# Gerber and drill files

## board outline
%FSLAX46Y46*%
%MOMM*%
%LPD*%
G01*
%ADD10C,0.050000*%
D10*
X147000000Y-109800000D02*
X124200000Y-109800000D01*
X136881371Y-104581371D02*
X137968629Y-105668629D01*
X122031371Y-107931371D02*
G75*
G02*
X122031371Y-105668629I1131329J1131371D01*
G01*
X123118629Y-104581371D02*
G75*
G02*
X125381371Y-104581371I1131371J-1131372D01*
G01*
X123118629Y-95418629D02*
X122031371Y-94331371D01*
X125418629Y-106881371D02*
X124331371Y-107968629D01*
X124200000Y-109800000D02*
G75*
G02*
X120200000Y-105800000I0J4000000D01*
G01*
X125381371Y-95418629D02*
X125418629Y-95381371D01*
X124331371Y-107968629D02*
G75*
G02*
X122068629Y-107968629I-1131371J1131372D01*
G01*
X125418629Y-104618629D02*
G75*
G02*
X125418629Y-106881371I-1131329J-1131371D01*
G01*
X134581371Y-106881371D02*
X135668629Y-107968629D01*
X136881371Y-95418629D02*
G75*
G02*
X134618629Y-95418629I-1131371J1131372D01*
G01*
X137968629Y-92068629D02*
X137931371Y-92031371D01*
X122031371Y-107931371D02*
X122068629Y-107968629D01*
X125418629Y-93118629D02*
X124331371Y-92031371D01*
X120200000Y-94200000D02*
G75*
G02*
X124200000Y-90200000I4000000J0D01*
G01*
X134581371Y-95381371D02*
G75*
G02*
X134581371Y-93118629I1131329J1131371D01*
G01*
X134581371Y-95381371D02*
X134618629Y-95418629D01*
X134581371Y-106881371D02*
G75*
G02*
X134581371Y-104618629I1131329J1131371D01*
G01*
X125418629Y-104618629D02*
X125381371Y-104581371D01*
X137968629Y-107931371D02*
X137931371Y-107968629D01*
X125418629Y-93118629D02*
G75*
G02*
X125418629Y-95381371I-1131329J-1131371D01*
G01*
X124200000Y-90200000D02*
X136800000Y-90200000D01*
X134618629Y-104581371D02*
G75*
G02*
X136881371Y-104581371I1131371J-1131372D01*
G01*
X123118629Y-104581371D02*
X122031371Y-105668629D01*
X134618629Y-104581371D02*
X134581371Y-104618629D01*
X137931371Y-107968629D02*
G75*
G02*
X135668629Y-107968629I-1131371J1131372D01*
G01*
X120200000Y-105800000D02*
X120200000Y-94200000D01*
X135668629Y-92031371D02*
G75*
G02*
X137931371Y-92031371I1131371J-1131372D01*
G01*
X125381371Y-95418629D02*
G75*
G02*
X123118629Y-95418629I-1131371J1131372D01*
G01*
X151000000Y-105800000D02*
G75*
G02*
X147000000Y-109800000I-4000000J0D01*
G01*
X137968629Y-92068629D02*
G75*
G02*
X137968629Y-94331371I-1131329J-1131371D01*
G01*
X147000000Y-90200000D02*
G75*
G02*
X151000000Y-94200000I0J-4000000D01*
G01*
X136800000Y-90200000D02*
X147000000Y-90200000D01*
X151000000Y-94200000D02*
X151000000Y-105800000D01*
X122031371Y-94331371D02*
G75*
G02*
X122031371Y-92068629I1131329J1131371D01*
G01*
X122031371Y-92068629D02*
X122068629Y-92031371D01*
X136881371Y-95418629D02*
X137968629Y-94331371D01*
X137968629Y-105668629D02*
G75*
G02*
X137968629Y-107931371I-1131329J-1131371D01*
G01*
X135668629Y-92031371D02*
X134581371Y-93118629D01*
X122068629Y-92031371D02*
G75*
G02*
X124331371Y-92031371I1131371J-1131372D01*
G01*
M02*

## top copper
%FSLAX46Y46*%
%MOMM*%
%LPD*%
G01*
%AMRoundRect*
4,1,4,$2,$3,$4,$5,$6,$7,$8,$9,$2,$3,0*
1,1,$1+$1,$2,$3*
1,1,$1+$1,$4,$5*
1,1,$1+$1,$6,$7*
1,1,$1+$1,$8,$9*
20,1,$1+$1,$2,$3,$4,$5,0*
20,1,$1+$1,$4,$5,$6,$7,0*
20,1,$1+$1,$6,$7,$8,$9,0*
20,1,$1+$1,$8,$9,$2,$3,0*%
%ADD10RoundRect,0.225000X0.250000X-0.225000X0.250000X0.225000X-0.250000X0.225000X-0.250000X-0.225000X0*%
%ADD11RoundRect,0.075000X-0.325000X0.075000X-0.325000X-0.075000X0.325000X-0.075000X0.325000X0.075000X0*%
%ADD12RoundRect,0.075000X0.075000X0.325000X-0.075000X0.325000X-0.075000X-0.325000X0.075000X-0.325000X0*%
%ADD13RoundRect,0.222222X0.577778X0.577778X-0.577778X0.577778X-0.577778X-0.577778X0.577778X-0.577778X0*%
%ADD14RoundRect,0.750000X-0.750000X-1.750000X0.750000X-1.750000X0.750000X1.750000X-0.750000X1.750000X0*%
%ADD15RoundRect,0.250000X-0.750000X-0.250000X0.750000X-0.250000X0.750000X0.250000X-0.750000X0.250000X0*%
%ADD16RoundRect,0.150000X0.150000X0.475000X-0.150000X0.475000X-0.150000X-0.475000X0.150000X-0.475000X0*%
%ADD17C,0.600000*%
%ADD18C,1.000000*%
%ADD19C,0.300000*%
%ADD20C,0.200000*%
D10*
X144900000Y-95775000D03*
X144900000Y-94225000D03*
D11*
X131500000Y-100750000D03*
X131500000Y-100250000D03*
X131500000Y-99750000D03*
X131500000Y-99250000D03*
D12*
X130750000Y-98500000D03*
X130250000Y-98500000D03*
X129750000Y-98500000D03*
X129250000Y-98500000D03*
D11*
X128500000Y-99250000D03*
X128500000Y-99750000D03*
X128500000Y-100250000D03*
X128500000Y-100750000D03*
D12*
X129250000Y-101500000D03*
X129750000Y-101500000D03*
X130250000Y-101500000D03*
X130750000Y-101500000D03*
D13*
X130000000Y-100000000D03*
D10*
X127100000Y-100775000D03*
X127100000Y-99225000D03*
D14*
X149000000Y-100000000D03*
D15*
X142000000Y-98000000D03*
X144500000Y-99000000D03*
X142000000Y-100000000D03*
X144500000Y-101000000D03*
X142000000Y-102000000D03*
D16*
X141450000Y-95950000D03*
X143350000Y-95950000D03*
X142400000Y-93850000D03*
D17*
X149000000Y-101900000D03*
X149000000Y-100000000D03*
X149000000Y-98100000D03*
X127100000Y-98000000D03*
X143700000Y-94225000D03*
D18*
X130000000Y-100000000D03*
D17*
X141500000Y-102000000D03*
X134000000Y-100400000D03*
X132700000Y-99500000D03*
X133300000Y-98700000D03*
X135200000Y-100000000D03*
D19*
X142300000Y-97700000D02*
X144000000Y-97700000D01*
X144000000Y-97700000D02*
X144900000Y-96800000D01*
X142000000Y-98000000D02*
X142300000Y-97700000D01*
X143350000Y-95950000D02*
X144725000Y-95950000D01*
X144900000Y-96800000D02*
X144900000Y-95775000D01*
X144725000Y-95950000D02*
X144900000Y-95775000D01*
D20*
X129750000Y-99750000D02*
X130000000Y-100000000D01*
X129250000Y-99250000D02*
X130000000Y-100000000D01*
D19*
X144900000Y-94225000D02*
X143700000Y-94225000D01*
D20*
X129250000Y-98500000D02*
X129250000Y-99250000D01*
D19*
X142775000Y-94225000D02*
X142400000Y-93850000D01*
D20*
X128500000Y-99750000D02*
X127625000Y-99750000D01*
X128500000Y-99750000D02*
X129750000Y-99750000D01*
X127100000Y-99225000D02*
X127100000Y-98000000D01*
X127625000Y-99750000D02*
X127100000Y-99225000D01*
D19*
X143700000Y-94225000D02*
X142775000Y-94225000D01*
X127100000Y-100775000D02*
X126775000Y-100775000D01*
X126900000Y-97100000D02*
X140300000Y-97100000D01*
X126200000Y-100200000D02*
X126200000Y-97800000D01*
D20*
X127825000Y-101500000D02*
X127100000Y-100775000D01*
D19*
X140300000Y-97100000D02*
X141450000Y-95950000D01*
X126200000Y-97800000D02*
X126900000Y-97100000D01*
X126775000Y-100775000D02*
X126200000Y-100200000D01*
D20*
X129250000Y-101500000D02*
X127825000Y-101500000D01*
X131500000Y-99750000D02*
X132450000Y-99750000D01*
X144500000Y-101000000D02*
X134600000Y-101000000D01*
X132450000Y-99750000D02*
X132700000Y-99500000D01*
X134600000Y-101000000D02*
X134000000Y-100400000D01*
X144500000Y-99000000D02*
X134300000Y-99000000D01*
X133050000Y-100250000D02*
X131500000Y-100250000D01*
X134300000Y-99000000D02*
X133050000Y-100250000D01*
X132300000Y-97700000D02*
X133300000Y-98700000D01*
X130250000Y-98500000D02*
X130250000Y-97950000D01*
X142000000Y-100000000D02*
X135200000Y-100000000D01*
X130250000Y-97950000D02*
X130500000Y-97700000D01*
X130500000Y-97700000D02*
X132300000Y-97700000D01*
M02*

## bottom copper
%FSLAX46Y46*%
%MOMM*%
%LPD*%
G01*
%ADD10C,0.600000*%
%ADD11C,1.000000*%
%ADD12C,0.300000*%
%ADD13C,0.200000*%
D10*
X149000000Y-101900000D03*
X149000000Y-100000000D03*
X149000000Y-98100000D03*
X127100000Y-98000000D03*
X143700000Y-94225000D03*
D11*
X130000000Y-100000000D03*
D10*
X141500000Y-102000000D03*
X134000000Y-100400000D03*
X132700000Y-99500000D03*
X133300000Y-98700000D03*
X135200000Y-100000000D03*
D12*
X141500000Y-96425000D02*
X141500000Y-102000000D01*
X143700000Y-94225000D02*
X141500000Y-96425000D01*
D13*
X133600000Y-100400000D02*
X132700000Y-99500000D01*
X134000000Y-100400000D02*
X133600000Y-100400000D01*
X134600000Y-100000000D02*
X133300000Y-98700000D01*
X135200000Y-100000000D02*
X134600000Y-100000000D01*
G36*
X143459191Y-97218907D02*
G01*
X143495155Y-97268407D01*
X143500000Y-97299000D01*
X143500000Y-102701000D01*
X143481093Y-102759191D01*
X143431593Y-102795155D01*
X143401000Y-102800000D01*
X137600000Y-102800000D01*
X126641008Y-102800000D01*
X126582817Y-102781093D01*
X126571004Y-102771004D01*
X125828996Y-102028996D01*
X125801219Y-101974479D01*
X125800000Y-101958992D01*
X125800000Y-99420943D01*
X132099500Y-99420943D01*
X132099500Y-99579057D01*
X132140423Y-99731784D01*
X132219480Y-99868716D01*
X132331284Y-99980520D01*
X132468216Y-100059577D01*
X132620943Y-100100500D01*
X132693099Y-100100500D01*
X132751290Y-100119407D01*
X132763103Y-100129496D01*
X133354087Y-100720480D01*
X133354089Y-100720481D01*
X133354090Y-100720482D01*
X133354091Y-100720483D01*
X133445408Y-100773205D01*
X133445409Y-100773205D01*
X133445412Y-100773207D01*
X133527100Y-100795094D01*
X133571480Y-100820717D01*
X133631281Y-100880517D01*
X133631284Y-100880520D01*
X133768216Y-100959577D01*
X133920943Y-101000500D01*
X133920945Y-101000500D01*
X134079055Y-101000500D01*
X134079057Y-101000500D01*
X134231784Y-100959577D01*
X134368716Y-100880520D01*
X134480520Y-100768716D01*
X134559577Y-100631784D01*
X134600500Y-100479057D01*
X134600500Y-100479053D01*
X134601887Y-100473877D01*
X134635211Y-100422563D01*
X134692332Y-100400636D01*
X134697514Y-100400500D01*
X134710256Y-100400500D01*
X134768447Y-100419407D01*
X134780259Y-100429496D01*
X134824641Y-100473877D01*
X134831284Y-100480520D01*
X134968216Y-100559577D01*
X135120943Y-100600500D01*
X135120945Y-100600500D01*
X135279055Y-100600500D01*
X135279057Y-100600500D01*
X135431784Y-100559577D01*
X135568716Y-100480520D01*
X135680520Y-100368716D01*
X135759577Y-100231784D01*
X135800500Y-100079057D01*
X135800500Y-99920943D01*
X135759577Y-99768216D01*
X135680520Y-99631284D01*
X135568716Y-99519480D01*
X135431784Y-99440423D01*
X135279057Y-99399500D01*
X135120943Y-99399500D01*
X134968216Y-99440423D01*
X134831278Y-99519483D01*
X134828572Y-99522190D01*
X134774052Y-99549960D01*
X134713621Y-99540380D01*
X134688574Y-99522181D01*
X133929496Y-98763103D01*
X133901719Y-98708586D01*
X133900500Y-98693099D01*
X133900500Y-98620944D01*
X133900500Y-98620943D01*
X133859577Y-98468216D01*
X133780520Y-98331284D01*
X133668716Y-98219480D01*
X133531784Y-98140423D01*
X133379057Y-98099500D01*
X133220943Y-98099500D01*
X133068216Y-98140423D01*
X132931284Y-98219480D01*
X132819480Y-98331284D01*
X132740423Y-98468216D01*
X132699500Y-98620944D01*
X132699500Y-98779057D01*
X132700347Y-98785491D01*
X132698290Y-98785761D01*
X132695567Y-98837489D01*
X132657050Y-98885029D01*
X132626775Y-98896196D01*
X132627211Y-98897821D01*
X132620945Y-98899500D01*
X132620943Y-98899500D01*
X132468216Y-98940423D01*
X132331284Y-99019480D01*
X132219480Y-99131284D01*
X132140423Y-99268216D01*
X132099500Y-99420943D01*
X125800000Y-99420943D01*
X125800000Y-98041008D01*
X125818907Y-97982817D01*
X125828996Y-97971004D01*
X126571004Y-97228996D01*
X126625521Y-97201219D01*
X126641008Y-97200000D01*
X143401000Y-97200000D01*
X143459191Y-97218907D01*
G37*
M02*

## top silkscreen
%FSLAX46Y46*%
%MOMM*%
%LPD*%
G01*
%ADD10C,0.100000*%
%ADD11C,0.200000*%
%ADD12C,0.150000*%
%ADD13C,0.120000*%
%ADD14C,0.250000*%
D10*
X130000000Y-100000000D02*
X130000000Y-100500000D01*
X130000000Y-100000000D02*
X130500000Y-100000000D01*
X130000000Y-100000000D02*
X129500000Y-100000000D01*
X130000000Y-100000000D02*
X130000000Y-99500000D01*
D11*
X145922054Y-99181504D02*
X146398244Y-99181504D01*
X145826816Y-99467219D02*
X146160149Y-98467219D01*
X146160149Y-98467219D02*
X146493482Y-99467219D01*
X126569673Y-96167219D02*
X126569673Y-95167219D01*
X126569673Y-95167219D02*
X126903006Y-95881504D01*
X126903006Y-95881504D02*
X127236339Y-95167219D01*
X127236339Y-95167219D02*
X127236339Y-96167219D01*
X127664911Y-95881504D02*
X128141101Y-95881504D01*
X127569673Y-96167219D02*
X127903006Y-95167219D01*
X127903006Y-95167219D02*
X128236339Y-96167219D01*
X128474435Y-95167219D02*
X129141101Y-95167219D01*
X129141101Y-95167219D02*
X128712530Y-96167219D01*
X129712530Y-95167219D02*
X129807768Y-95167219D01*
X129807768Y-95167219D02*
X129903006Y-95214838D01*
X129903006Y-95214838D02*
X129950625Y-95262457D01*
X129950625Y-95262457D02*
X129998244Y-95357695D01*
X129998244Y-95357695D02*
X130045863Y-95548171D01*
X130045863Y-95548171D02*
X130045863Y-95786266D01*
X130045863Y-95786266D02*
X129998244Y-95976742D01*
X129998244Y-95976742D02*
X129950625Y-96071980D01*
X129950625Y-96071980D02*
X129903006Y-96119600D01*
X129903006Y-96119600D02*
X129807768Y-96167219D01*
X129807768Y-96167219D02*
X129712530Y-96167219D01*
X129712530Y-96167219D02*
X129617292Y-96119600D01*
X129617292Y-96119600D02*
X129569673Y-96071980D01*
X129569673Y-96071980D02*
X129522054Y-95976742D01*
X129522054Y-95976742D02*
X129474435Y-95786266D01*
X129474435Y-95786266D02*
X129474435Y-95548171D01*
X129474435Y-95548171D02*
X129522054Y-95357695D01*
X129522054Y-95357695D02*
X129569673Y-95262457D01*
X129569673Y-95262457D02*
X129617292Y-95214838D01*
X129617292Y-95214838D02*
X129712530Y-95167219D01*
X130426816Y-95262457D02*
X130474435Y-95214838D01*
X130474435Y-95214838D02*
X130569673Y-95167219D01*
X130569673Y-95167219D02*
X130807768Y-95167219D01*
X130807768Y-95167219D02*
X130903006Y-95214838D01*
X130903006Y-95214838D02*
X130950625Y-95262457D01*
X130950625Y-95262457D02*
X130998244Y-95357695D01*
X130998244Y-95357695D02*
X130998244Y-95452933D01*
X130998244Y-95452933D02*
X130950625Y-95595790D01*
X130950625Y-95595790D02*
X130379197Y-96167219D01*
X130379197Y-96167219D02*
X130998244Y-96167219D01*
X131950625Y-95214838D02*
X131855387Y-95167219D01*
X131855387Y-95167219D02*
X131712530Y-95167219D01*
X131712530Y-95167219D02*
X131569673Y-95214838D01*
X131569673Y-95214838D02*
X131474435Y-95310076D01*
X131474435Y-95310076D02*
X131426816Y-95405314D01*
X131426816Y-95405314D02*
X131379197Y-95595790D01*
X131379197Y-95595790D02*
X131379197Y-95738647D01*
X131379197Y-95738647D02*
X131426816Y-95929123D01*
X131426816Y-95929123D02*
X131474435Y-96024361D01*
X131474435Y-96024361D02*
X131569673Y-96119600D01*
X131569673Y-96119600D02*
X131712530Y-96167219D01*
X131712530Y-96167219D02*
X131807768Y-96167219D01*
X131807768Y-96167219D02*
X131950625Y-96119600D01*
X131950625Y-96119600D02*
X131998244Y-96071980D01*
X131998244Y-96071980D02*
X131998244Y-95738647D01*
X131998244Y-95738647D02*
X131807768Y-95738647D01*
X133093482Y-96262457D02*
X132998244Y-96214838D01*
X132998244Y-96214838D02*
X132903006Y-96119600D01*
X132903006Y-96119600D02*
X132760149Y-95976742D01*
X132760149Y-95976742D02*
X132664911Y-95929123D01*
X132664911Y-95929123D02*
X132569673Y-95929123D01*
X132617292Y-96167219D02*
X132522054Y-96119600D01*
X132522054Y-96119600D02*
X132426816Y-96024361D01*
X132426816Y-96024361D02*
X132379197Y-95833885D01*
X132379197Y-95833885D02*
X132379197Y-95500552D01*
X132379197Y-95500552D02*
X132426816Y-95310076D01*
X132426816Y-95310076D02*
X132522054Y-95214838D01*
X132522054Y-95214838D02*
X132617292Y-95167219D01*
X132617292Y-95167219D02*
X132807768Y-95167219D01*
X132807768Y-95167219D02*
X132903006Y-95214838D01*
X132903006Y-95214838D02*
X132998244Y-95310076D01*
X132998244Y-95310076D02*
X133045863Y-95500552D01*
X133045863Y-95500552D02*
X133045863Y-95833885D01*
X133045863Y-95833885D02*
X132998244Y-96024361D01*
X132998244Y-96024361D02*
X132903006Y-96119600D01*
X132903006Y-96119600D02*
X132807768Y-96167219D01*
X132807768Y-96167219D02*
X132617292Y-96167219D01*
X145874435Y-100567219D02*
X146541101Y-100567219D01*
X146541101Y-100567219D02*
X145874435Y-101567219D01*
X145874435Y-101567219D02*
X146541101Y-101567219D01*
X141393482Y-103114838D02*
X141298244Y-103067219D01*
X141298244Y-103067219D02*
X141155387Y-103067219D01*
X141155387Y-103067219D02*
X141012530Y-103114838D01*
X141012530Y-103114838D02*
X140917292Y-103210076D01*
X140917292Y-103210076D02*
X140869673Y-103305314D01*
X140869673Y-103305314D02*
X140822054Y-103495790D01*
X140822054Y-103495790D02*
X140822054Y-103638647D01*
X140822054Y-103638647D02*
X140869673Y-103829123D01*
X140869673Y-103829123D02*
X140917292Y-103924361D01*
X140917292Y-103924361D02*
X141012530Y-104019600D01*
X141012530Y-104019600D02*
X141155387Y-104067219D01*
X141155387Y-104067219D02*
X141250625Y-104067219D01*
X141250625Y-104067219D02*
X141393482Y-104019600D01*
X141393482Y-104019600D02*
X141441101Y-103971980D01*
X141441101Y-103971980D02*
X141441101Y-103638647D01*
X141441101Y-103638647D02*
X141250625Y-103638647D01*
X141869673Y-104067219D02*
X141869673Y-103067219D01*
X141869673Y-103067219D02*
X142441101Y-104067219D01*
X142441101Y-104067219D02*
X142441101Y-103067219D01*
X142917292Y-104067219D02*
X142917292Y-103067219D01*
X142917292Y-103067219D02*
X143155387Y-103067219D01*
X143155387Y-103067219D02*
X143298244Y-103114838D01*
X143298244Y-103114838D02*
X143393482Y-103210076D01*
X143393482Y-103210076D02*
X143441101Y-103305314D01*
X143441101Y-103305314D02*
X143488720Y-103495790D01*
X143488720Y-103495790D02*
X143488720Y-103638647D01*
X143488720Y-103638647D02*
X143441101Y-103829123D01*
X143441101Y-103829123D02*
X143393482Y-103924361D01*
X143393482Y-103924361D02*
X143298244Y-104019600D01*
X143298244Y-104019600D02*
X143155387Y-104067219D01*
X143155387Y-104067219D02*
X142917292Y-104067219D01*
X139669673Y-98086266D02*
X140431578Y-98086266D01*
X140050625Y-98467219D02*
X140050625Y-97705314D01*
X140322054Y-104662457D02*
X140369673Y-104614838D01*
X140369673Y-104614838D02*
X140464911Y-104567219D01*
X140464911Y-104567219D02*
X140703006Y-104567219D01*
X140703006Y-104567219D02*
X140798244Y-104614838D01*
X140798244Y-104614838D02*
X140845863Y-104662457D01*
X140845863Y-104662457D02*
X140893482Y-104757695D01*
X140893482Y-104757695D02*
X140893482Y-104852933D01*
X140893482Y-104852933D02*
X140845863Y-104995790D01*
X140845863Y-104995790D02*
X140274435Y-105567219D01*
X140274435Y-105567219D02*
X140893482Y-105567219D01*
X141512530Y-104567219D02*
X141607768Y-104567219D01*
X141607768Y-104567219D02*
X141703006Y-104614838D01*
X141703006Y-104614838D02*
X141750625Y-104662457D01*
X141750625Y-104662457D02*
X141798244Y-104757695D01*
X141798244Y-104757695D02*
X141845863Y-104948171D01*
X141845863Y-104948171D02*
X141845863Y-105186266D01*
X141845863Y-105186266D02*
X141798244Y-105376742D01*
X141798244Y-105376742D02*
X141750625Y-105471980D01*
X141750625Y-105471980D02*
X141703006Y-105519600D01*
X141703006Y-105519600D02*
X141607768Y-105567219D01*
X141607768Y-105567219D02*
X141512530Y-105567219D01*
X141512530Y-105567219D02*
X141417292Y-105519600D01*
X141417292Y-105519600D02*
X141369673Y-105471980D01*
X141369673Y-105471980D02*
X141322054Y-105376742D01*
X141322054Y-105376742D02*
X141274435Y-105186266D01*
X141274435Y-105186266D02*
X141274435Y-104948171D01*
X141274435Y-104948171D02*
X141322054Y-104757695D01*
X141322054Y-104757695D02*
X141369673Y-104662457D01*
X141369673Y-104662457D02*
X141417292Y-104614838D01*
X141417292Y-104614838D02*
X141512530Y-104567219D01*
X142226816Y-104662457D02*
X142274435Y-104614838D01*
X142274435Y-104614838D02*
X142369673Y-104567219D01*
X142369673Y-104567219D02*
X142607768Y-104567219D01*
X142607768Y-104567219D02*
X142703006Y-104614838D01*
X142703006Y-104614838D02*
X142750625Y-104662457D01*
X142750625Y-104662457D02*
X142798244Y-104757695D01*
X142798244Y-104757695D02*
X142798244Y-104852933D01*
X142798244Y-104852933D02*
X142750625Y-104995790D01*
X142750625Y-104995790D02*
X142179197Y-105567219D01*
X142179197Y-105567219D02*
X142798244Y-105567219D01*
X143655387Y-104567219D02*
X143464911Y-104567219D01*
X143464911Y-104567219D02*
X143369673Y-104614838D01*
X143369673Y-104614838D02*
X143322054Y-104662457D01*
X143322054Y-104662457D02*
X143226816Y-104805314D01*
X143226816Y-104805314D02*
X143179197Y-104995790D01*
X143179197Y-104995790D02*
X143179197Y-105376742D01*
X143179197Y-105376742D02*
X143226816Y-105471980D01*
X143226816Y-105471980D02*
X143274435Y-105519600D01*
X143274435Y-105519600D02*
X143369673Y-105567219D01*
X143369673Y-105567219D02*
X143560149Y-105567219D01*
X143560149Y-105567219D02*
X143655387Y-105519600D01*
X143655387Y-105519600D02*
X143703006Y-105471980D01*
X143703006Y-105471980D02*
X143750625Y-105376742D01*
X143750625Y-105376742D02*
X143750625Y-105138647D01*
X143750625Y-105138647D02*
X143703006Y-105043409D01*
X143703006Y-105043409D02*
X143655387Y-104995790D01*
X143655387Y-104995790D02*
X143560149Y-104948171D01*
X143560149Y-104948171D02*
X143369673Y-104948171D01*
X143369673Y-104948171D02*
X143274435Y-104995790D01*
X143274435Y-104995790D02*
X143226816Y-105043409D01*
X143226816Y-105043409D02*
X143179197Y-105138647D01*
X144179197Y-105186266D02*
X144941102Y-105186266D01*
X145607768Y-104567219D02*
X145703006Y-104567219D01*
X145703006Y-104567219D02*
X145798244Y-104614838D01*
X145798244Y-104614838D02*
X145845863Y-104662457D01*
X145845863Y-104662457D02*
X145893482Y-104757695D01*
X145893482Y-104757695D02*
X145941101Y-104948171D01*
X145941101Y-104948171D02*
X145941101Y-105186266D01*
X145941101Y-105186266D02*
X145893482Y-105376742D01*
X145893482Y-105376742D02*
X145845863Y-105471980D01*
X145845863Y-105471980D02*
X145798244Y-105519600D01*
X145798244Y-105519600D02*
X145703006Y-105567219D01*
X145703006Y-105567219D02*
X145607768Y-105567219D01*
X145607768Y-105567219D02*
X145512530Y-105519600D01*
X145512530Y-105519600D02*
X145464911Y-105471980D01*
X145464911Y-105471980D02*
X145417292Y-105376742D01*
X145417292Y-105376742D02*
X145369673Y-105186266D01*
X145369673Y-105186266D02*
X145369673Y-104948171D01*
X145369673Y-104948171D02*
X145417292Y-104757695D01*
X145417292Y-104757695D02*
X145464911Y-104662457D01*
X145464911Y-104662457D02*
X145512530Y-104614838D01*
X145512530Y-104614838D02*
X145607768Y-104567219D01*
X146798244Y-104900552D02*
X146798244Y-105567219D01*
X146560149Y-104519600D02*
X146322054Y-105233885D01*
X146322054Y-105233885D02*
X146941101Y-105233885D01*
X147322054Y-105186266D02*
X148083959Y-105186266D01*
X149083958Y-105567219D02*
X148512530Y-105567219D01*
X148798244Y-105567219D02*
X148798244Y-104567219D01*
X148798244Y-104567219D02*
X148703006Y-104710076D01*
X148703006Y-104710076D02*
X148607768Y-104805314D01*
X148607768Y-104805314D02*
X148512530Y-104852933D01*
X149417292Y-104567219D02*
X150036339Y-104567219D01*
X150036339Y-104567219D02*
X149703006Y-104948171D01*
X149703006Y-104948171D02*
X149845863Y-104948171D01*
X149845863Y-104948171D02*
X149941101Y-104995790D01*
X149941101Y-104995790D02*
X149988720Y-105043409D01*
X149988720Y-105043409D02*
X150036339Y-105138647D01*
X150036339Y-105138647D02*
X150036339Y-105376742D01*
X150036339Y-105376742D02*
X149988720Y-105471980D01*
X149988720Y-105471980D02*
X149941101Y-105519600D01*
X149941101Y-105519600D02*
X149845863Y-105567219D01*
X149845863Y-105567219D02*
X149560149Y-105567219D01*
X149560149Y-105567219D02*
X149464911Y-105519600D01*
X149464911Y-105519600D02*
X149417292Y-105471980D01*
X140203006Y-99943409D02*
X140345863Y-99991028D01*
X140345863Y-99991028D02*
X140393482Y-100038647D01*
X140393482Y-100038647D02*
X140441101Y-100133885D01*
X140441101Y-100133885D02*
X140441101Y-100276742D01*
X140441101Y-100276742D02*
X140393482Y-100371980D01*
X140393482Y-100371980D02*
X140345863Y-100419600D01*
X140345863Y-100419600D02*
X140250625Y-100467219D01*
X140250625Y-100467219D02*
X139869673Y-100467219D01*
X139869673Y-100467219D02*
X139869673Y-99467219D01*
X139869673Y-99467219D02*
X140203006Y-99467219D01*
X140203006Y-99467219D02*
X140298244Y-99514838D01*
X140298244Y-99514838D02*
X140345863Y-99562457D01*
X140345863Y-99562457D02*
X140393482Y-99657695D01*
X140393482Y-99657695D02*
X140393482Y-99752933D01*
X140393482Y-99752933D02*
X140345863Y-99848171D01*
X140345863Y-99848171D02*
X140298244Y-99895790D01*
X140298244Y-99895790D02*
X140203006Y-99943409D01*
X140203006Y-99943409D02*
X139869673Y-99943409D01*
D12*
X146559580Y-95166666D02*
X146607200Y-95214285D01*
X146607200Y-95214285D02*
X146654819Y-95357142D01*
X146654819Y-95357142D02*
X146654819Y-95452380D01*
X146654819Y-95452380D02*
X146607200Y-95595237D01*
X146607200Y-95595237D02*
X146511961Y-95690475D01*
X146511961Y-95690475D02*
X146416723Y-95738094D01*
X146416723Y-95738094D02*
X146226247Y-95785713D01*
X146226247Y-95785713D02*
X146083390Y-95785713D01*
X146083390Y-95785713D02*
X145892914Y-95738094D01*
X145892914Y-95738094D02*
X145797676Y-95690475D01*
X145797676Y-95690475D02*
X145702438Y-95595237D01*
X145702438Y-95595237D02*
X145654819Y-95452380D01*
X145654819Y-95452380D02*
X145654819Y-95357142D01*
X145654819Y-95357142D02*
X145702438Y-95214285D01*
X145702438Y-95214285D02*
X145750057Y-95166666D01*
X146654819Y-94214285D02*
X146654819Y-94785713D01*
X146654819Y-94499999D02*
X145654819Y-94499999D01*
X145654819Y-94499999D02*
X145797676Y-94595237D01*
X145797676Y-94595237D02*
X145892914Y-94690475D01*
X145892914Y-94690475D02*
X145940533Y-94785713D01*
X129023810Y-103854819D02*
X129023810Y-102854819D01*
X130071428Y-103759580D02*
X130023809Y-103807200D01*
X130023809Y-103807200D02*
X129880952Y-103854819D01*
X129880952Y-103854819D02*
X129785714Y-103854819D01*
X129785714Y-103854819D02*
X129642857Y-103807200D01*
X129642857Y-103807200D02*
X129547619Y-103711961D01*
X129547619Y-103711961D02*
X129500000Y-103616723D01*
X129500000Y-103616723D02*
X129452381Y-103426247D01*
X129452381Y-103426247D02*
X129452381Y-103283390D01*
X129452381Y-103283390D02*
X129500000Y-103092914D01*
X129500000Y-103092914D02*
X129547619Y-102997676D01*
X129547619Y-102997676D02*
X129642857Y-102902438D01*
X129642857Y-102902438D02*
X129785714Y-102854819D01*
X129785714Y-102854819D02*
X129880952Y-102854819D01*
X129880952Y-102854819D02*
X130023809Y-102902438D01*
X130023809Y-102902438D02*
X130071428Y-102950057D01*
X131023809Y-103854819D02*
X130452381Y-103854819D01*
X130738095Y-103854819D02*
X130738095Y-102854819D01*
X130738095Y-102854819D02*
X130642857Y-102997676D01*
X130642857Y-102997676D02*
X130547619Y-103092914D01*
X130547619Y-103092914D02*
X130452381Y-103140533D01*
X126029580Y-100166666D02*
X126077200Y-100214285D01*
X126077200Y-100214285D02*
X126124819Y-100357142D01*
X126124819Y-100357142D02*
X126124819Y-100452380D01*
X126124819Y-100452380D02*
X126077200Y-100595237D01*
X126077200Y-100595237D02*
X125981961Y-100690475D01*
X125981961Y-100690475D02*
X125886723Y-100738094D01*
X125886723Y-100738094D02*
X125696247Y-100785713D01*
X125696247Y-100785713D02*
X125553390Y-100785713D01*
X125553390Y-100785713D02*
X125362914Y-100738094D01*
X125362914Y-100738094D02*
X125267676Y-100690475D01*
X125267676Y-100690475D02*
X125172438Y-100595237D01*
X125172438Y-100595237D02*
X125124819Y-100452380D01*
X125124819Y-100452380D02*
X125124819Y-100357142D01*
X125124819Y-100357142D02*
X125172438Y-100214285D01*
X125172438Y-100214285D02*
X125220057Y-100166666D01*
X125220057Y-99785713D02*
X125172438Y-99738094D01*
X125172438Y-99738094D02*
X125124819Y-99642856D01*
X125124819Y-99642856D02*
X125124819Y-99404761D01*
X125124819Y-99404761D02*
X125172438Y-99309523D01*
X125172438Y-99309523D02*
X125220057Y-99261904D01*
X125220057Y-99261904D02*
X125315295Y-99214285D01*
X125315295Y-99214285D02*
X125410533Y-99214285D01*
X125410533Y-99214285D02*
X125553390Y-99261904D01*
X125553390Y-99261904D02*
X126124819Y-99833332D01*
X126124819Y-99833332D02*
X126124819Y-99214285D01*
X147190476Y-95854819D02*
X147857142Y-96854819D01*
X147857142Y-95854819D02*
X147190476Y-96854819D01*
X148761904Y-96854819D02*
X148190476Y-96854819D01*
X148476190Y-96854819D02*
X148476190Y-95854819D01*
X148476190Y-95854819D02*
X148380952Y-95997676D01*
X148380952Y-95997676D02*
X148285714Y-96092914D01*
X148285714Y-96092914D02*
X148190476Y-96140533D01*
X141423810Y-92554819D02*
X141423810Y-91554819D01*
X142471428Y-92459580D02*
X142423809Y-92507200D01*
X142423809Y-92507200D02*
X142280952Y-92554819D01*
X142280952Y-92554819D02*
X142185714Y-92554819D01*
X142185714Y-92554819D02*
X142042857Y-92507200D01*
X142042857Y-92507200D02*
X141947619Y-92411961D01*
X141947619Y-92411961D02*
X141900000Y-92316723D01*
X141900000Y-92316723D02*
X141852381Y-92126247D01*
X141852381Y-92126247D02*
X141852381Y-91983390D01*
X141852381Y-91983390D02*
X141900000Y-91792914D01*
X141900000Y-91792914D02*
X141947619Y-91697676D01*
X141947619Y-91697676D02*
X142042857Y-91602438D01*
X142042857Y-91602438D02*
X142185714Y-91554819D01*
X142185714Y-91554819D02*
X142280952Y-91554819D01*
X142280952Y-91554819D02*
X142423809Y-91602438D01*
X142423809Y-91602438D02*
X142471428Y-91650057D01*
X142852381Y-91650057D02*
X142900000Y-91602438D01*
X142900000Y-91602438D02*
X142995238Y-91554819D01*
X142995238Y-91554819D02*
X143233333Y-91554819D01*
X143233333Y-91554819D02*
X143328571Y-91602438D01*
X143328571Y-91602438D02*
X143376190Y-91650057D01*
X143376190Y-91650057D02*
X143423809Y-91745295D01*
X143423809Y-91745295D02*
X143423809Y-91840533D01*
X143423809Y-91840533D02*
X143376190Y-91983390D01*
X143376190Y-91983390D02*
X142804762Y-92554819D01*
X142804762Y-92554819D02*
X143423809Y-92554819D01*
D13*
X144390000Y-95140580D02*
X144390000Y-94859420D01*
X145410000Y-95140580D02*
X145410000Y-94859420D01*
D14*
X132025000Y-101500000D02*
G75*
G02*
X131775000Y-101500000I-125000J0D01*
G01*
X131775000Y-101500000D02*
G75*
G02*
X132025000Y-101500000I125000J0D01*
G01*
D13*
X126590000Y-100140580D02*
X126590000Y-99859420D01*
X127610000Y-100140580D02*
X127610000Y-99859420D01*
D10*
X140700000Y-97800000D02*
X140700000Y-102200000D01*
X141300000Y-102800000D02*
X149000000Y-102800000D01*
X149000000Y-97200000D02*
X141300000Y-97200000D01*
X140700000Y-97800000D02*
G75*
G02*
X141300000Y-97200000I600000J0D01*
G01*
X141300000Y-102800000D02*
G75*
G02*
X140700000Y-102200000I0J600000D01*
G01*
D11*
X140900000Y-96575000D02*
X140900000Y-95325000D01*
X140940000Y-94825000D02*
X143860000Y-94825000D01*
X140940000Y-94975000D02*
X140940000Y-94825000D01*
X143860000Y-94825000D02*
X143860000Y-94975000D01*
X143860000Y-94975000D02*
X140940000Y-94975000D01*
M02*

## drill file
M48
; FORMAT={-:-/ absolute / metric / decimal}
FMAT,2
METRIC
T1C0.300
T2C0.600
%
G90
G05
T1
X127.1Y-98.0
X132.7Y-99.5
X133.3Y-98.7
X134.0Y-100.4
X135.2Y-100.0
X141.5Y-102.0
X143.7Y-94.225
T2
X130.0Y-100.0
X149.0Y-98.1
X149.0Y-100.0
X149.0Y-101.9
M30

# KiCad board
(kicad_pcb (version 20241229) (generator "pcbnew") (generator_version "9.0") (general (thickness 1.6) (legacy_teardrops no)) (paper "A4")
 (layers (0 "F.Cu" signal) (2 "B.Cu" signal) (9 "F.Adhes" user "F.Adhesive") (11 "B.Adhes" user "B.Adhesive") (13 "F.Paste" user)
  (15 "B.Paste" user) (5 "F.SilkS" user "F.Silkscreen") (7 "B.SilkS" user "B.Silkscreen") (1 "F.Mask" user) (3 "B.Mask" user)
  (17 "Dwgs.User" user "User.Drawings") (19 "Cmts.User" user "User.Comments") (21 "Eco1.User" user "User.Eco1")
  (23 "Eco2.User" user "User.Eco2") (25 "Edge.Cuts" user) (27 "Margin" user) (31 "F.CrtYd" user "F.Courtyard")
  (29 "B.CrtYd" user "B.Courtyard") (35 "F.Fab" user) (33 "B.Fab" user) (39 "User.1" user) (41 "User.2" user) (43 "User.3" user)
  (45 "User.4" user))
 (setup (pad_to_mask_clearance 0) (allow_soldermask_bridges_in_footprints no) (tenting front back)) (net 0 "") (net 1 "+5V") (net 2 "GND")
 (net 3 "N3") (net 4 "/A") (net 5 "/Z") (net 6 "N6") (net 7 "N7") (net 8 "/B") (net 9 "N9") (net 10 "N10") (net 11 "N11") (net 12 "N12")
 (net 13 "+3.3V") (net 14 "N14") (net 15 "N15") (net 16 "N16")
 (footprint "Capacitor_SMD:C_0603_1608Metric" (layer "F.Cu") (at 144.9 95 90)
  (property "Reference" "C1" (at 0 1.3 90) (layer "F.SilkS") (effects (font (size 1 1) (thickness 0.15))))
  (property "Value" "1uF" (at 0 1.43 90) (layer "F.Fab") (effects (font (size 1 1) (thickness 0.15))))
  (fp_line (start -0.14058 -0.51) (end 0.14058 -0.51) (stroke (width 0.12) (type solid)) (layer "F.SilkS"))
  (fp_line (start -0.14058 0.51) (end 0.14058 0.51) (stroke (width 0.12) (type solid)) (layer "F.SilkS"))
  (pad "1" smd roundrect (at -0.775 0 90) (size 0.9 0.95) (layers "F.Cu" "F.Mask" "F.Paste") (roundrect_rratio 0.25) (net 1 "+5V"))
  (pad "2" smd roundrect (at 0.775 0 90) (size 0.9 0.95) (layers "F.Cu" "F.Mask" "F.Paste") (roundrect_rratio 0.25) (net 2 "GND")))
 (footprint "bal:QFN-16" (layer "F.Cu") (at 130 100 180)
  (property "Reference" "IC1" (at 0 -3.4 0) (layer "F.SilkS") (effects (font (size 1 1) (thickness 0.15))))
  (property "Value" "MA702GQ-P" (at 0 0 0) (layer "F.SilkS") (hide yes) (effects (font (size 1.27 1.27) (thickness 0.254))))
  (fp_circle (center -1.9 -1.5) (end -1.9 -1.375) (stroke (width 0.25) (type solid)) (fill no) (layer "F.SilkS"))
  (pad "1" smd roundrect (at -1.5 -0.75 270) (size 0.3 0.8) (layers "F.Cu" "F.Mask" "F.Paste") (roundrect_rratio 0.25) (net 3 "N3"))
  (pad "2" smd roundrect (at -1.5 -0.25 270) (size 0.3 0.8) (layers "F.Cu" "F.Mask" "F.Paste") (roundrect_rratio 0.25) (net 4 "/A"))
  (pad "3" smd roundrect (at -1.5 0.25 270) (size 0.3 0.8) (layers "F.Cu" "F.Mask" "F.Paste") (roundrect_rratio 0.25) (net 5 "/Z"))
  (pad "4" smd roundrect (at -1.5 0.75 270) (size 0.3 0.8) (layers "F.Cu" "F.Mask" "F.Paste") (roundrect_rratio 0.25) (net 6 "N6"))
  (pad "5" smd roundrect (at -0.75 1.5 180) (size 0.3 0.8) (layers "F.Cu" "F.Mask" "F.Paste") (roundrect_rratio 0.25) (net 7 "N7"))
  (pad "6" smd roundrect (at -0.25 1.5 180) (size 0.3 0.8) (layers "F.Cu" "F.Mask" "F.Paste") (roundrect_rratio 0.25) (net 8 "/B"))
  (pad "7" smd roundrect (at 0.25 1.5 180) (size 0.3 0.8) (layers "F.Cu" "F.Mask" "F.Paste") (roundrect_rratio 0.25) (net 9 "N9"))
  (pad "8" smd roundrect (at 0.75 1.5 180) (size 0.3 0.8) (layers "F.Cu" "F.Mask" "F.Paste") (roundrect_rratio 0.25) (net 2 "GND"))
  (pad "9" smd roundrect (at 1.5 0.75 270) (size 0.3 0.8) (layers "F.Cu" "F.Mask" "F.Paste") (roundrect_rratio 0.25) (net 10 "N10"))
  (pad "10" smd roundrect (at 1.5 0.25 270) (size 0.3 0.8) (layers "F.Cu" "F.Mask" "F.Paste") (roundrect_rratio 0.25) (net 2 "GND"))
  (pad "11" smd roundrect (at 1.5 -0.25 270) (size 0.3 0.8) (layers "F.Cu" "F.Mask" "F.Paste") (roundrect_rratio 0.25) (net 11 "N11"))
  (pad "12" smd roundrect (at 1.5 -0.75 270) (size 0.3 0.8) (layers "F.Cu" "F.Mask" "F.Paste") (roundrect_rratio 0.25) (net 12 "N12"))
  (pad "13" smd roundrect (at 0.75 -1.5 180) (size 0.3 0.8) (layers "F.Cu" "F.Mask" "F.Paste") (roundrect_rratio 0.25) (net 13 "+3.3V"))
  (pad "14" smd roundrect (at 0.25 -1.5 180) (size 0.3 0.8) (layers "F.Cu" "F.Mask" "F.Paste") (roundrect_rratio 0.25) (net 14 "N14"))
  (pad "15" smd roundrect (at -0.25 -1.5 180) (size 0.3 0.8) (layers "F.Cu" "F.Mask" "F.Paste") (roundrect_rratio 0.25) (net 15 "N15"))
  (pad "16" smd roundrect (at -0.75 -1.5 180) (size 0.3 0.8) (layers "F.Cu" "F.Mask" "F.Paste") (roundrect_rratio 0.25) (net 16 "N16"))
  (pad "17" smd roundrect (at 0 0 180) (size 1.6 1.6) (layers "F.Cu" "F.Mask" "F.Paste") (roundrect_rratio 0.1388888889) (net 2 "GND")))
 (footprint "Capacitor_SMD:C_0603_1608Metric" (layer "F.Cu") (at 127.1 100 90)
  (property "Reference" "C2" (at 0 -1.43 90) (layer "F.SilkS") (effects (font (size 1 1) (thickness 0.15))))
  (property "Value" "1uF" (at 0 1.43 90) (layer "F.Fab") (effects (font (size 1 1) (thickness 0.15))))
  (fp_line (start -0.14058 -0.51) (end 0.14058 -0.51) (stroke (width 0.12) (type solid)) (layer "F.SilkS"))
  (fp_line (start -0.14058 0.51) (end 0.14058 0.51) (stroke (width 0.12) (type solid)) (layer "F.SilkS"))
  (pad "1" smd roundrect (at -0.775 0 90) (size 0.9 0.95) (layers "F.Cu" "F.Mask" "F.Paste") (roundrect_rratio 0.25) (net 13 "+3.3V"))
  (pad "2" smd roundrect (at 0.775 0 90) (size 0.9 0.95) (layers "F.Cu" "F.Mask" "F.Paste") (roundrect_rratio 0.25) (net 2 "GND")))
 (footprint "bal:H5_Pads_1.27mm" (layer "F.Cu") (at 142 98)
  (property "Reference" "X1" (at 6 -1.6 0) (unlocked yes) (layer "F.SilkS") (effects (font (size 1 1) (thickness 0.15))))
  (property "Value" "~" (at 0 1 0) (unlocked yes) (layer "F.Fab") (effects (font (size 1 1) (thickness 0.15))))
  (fp_line (start -1.3 -0.2) (end -1.3 4.2) (stroke (width 0.1) (type default)) (layer "F.SilkS"))
  (fp_line (start -0.7 4.8) (end 7 4.8) (stroke (width 0.1) (type default)) (layer "F.SilkS"))
  (fp_line (start 7 -0.8) (end -0.7 -0.8) (stroke (width 0.1) (type default)) (layer "F.SilkS"))
  (fp_arc (start -1.3 -0.2) (mid -1.124264 -0.624264) (end -0.7 -0.8) (stroke (width 0.1) (type default)) (layer "F.SilkS"))
  (fp_arc (start -0.7 4.8) (mid -1.124264 4.624264) (end -1.3 4.2) (stroke (width 0.1) (type default)) (layer "F.SilkS"))
  (pad "" smd roundrect (at 7 2) (size 3 5) (layers "F.Cu" "F.Mask" "F.Paste") (roundrect_rratio 0.25) (thermal_bridge_angle 45))
  (pad "1" smd roundrect (at 0 0) (size 2 1) (layers "F.Cu" "F.Mask" "F.Paste") (roundrect_rratio 0.25) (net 1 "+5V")
   (thermal_bridge_angle 45))
  (pad "2" smd roundrect (at 2.5 1) (size 2 1) (layers "F.Cu" "F.Mask" "F.Paste") (roundrect_rratio 0.25) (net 4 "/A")
   (thermal_bridge_angle 45))
  (pad "3" smd roundrect (at 0 2) (size 2 1) (layers "F.Cu" "F.Mask" "F.Paste") (roundrect_rratio 0.25) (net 8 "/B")
   (thermal_bridge_angle 45))
  (pad "4" smd roundrect (at 2.5 3) (size 2 1) (layers "F.Cu" "F.Mask" "F.Paste") (roundrect_rratio 0.25) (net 5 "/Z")
   (thermal_bridge_angle 45))
  (pad "5" smd roundrect (at 0 4) (size 2 1) (layers "F.Cu" "F.Mask" "F.Paste") (roundrect_rratio 0.25) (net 2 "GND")
   (thermal_bridge_angle 45)))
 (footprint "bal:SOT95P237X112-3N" (layer "F.Cu") (at 142.4 94.9 90)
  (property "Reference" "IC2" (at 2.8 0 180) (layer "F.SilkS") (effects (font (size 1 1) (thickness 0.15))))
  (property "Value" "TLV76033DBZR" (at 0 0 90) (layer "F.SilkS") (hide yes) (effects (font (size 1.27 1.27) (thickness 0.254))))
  (fp_line (start -1.675 -1.5) (end -0.425 -1.5) (stroke (width 0.2) (type solid)) (layer "F.SilkS"))
  (fp_line (start 0.075 -1.46) (end 0.075 1.46) (stroke (width 0.2) (type solid)) (layer "F.SilkS"))
  (fp_line (start -0.075 -1.46) (end 0.075 -1.46) (stroke (width 0.2) (type solid)) (layer "F.SilkS"))
  (fp_line (start 0.075 1.46) (end -0.075 1.46) (stroke (width 0.2) (type solid)) (layer "F.SilkS"))
  (fp_line (start -0.075 1.46) (end -0.075 -1.46) (stroke (width 0.2) (type solid)) (layer "F.SilkS"))
  (pad "1" smd roundrect (at -1.05 -0.95 180) (size 0.6 1.25) (layers "F.Cu" "F.Mask" "F.Paste") (roundrect_rratio 0.25) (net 13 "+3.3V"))
  (pad "2" smd roundrect (at -1.05 0.95 180) (size 0.6 1.25) (layers "F.Cu" "F.Mask" "F.Paste") (roundrect_rratio 0.25) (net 1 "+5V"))
  (pad "3" smd roundrect (at 1.05 0 180) (size 0.6 1.25) (layers "F.Cu" "F.Mask" "F.Paste") (roundrect_rratio 0.25) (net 2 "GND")))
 (gr_line (start 130 100) (end 130 100.5) (stroke (width 0.1) (type default)) (layer "F.SilkS"))
 (gr_line (start 130 100) (end 130.5 100) (stroke (width 0.1) (type default)) (layer "F.SilkS"))
 (gr_line (start 130 100) (end 129.5 100) (stroke (width 0.1) (type default)) (layer "F.SilkS"))
 (gr_line (start 130 100) (end 130 99.5) (stroke (width 0.1) (type default)) (layer "F.SilkS"))
 (gr_line (start 147 109.8) (end 124.2 109.8) (stroke (width 0.05) (type default)) (layer "Edge.Cuts"))
 (gr_line (start 136.881371 104.581371) (end 137.968629 105.668629) (stroke (width 0.05) (type default)) (layer "Edge.Cuts"))
 (gr_arc (start 122.031371 107.931371) (mid 121.562729 106.8) (end 122.031371 105.668629) (stroke (width 0.05) (type default))
  (layer "Edge.Cuts"))
 (gr_arc (start 123.118629 104.581371) (mid 124.25 104.112742) (end 125.381371 104.581371) (stroke (width 0.05) (type default))
  (layer "Edge.Cuts"))
 (gr_line (start 123.118629 95.418629) (end 122.031371 94.331371) (stroke (width 0.05) (type default)) (layer "Edge.Cuts"))
 (gr_line (start 125.418629 106.881371) (end 124.331371 107.968629) (stroke (width 0.05) (type default)) (layer "Edge.Cuts"))
 (gr_arc (start 124.2 109.8) (mid 121.371573 108.628427) (end 120.2 105.8) (stroke (width 0.05) (type default)) (layer "Edge.Cuts"))
 (gr_line (start 125.381371 95.418629) (end 125.418629 95.381371) (stroke (width 0.05) (type default)) (layer "Edge.Cuts"))
 (gr_arc (start 124.331371 107.968629) (mid 123.2 108.437258) (end 122.068629 107.968629) (stroke (width 0.05) (type default))
  (layer "Edge.Cuts"))
 (gr_arc (start 125.418629 104.618629) (mid 125.887258 105.75) (end 125.418629 106.881371) (stroke (width 0.05) (type default))
  (layer "Edge.Cuts"))
 (gr_line (start 134.581371 106.881371) (end 135.668629 107.968629) (stroke (width 0.05) (type default)) (layer "Edge.Cuts"))
 (gr_arc (start 136.881371 95.418629) (mid 135.75 95.887258) (end 134.618629 95.418629) (stroke (width 0.05) (type default))
  (layer "Edge.Cuts"))
 (gr_line (start 137.968629 92.068629) (end 137.931371 92.031371) (stroke (width 0.05) (type default)) (layer "Edge.Cuts"))
 (gr_line (start 122.031371 107.931371) (end 122.068629 107.968629) (stroke (width 0.05) (type default)) (layer "Edge.Cuts"))
 (gr_line (start 125.418629 93.118629) (end 124.331371 92.031371) (stroke (width 0.05) (type default)) (layer "Edge.Cuts"))
 (gr_arc (start 120.2 94.2) (mid 121.371573 91.371573) (end 124.2 90.2) (stroke (width 0.05) (type default)) (layer "Edge.Cuts"))
 (gr_arc (start 134.581371 95.381371) (mid 134.112729 94.25) (end 134.581371 93.118629) (stroke (width 0.05) (type default))
  (layer "Edge.Cuts"))
 (gr_line (start 134.581371 95.381371) (end 134.618629 95.418629) (stroke (width 0.05) (type default)) (layer "Edge.Cuts"))
 (gr_arc (start 134.581371 106.881371) (mid 134.112729 105.75) (end 134.581371 104.618629) (stroke (width 0.05) (type default))
  (layer "Edge.Cuts"))
 (gr_line (start 125.418629 104.618629) (end 125.381371 104.581371) (stroke (width 0.05) (type default)) (layer "Edge.Cuts"))
 (gr_line (start 137.968629 107.931371) (end 137.931371 107.968629) (stroke (width 0.05) (type default)) (layer "Edge.Cuts"))
 (gr_arc (start 125.418629 93.118629) (mid 125.887258 94.25) (end 125.418629 95.381371) (stroke (width 0.05) (type default))
  (layer "Edge.Cuts"))
 (gr_line (start 124.2 90.2) (end 136.8 90.2) (stroke (width 0.05) (type default)) (layer "Edge.Cuts"))
 (gr_arc (start 134.618629 104.581371) (mid 135.75 104.112742) (end 136.881371 104.581371) (stroke (width 0.05) (type default))
  (layer "Edge.Cuts"))
 (gr_line (start 123.118629 104.581371) (end 122.031371 105.668629) (stroke (width 0.05) (type default)) (layer "Edge.Cuts"))
 (gr_line (start 134.618629 104.581371) (end 134.581371 104.618629) (stroke (width 0.05) (type default)) (layer "Edge.Cuts"))
 (gr_arc (start 137.931371 107.968629) (mid 136.8 108.437258) (end 135.668629 107.968629) (stroke (width 0.05) (type default))
  (layer "Edge.Cuts"))
 (gr_line (start 120.2 105.8) (end 120.2 94.2) (stroke (width 0.05) (type default)) (layer "Edge.Cuts"))
 (gr_arc (start 135.668629 92.031371) (mid 136.8 91.562742) (end 137.931371 92.031371) (stroke (width 0.05) (type default))
  (layer "Edge.Cuts"))
 (gr_arc (start 125.381371 95.418629) (mid 124.25 95.887258) (end 123.118629 95.418629) (stroke (width 0.05) (type default))
  (layer "Edge.Cuts"))
 (gr_arc (start 151 105.8) (mid 149.828427 108.628427) (end 147 109.8) (stroke (width 0.05) (type default)) (layer "Edge.Cuts"))
 (gr_arc (start 137.968629 92.068629) (mid 138.437258 93.2) (end 137.968629 94.331371) (stroke (width 0.05) (type default))
  (layer "Edge.Cuts"))
 (gr_arc (start 147 90.2) (mid 149.828427 91.371573) (end 151 94.2) (stroke (width 0.05) (type default)) (layer "Edge.Cuts"))
 (gr_line (start 136.8 90.2) (end 147 90.2) (stroke (width 0.05) (type default)) (layer "Edge.Cuts"))
 (gr_line (start 151 94.2) (end 151 105.8) (stroke (width 0.05) (type default)) (layer "Edge.Cuts"))
 (gr_arc (start 122.031371 94.331371) (mid 121.562729 93.2) (end 122.031371 92.068629) (stroke (width 0.05) (type default))
  (layer "Edge.Cuts"))
 (gr_line (start 122.031371 92.068629) (end 122.068629 92.031371) (stroke (width 0.05) (type default)) (layer "Edge.Cuts"))
 (gr_line (start 136.881371 95.418629) (end 137.968629 94.331371) (stroke (width 0.05) (type default)) (layer "Edge.Cuts"))
 (gr_arc (start 137.968629 105.668629) (mid 138.437271 106.8) (end 137.968629 107.931371) (stroke (width 0.05) (type default))
  (layer "Edge.Cuts"))
 (gr_line (start 135.668629 92.031371) (end 134.581371 93.118629) (stroke (width 0.05) (type default)) (layer "Edge.Cuts"))
 (gr_arc (start 122.068629 92.031371) (mid 123.2 91.562742) (end 124.331371 92.031371) (stroke (width 0.05) (type default))
  (layer "Edge.Cuts"))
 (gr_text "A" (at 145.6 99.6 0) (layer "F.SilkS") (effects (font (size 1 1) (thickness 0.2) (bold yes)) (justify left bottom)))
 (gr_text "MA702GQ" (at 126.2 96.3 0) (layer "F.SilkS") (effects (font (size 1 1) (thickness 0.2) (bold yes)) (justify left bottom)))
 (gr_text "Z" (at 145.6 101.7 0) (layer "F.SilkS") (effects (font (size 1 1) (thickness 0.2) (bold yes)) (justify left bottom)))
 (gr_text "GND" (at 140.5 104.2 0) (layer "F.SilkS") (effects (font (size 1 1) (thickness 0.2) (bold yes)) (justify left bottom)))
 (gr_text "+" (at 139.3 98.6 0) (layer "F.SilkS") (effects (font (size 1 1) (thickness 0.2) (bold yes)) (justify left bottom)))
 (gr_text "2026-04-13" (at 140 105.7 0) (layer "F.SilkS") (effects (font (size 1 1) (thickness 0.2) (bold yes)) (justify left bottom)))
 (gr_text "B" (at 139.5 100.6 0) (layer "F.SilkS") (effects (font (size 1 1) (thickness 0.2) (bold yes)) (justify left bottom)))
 (via (at 149 101.9) (size 0.6) (drill 0.6) (layers "F.Cu" "B.Cu") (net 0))
 (via (at 149 100) (size 0.6) (drill 0.6) (layers "F.Cu" "B.Cu") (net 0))
 (via (at 149 98.1) (size 0.6) (drill 0.6) (layers "F.Cu" "B.Cu") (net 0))
 (segment (start 142.3 97.7) (end 144 97.7) (width 0.3) (layer "F.Cu") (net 1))
 (segment (start 144 97.7) (end 144.9 96.8) (width 0.3) (layer "F.Cu") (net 1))
 (segment (start 142 98) (end 142.3 97.7) (width 0.3) (layer "F.Cu") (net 1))
 (segment (start 143.35 95.95) (end 144.725 95.95) (width 0.3) (layer "F.Cu") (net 1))
 (segment (start 144.9 96.8) (end 144.9 95.775) (width 0.3) (layer "F.Cu") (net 1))
 (segment (start 144.725 95.95) (end 144.9 95.775) (width 0.3) (layer "F.Cu") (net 1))
 (segment (start 129.75 99.75) (end 130 100) (width 0.2) (layer "F.Cu") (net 2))
 (segment (start 129.25 99.25) (end 130 100) (width 0.2) (layer "F.Cu") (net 2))
 (segment (start 144.9 94.225) (end 143.7 94.225) (width 0.3) (layer "F.Cu") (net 2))
 (segment (start 129.25 98.5) (end 129.25 99.25) (width 0.2) (layer "F.Cu") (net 2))
 (segment (start 142.775 94.225) (end 142.4 93.85) (width 0.3) (layer "F.Cu") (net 2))
 (segment (start 128.5 99.75) (end 127.625 99.75) (width 0.2) (layer "F.Cu") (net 2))
 (segment (start 128.5 99.75) (end 129.75 99.75) (width 0.2) (layer "F.Cu") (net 2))
 (segment (start 127.1 99.225) (end 127.1 98) (width 0.2) (layer "F.Cu") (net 2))
 (segment (start 127.625 99.75) (end 127.1 99.225) (width 0.2) (layer "F.Cu") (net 2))
 (segment (start 143.7 94.225) (end 142.775 94.225) (width 0.3) (layer "F.Cu") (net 2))
 (via (at 127.1 98) (size 0.6) (drill 0.3) (layers "F.Cu" "B.Cu") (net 2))
 (via (at 143.7 94.225) (size 0.6) (drill 0.3) (layers "F.Cu" "B.Cu") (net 2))
 (via (at 130 100) (size 1) (drill 0.6) (layers "F.Cu" "B.Cu") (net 2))
 (via (at 141.5 102) (size 0.6) (drill 0.3) (layers "F.Cu" "B.Cu") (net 2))
 (segment (start 141.5 96.425) (end 141.5 102) (width 0.3) (layer "B.Cu") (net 2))
 (segment (start 143.7 94.225) (end 141.5 96.425) (width 0.3) (layer "B.Cu") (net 2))
 (segment (start 127.1 100.775) (end 126.775 100.775) (width 0.3) (layer "F.Cu") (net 13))
 (segment (start 126.9 97.1) (end 140.3 97.1) (width 0.3) (layer "F.Cu") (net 13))
 (segment (start 126.2 100.2) (end 126.2 97.8) (width 0.3) (layer "F.Cu") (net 13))
 (segment (start 127.825 101.5) (end 127.1 100.775) (width 0.2) (layer "F.Cu") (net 13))
 (segment (start 140.3 97.1) (end 141.45 95.95) (width 0.3) (layer "F.Cu") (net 13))
 (segment (start 126.2 97.8) (end 126.9 97.1) (width 0.3) (layer "F.Cu") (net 13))
 (segment (start 126.775 100.775) (end 126.2 100.2) (width 0.3) (layer "F.Cu") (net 13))
 (segment (start 129.25 101.5) (end 127.825 101.5) (width 0.2) (layer "F.Cu") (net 13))
 (segment (start 131.5 99.75) (end 132.45 99.75) (width 0.2) (layer "F.Cu") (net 5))
 (segment (start 144.5 101) (end 134.6 101) (width 0.2) (layer "F.Cu") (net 5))
 (segment (start 132.45 99.75) (end 132.7 99.5) (width 0.2) (layer "F.Cu") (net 5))
 (segment (start 134.6 101) (end 134 100.4) (width 0.2) (layer "F.Cu") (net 5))
 (via (at 134 100.4) (size 0.6) (drill 0.3) (layers "F.Cu" "B.Cu") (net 5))
 (via (at 132.7 99.5) (size 0.6) (drill 0.3) (layers "F.Cu" "B.Cu") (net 5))
 (segment (start 133.6 100.4) (end 132.7 99.5) (width 0.2) (layer "B.Cu") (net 5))
 (segment (start 134 100.4) (end 133.6 100.4) (width 0.2) (layer "B.Cu") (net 5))
 (segment (start 144.5 99) (end 134.3 99) (width 0.2) (layer "F.Cu") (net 4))
 (segment (start 133.05 100.25) (end 131.5 100.25) (width 0.2) (layer "F.Cu") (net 4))
 (segment (start 134.3 99) (end 133.05 100.25) (width 0.2) (layer "F.Cu") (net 4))
 (segment (start 132.3 97.7) (end 133.3 98.7) (width 0.2) (layer "F.Cu") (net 8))
 (segment (start 130.25 98.5) (end 130.25 97.95) (width 0.2) (layer "F.Cu") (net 8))
 (segment (start 142 100) (end 135.2 100) (width 0.2) (layer "F.Cu") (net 8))
 (segment (start 130.25 97.95) (end 130.5 97.7) (width 0.2) (layer "F.Cu") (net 8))
 (segment (start 130.5 97.7) (end 132.3 97.7) (width 0.2) (layer "F.Cu") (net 8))
 (via (at 133.3 98.7) (size 0.6) (drill 0.3) (layers "F.Cu" "B.Cu") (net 8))
 (via (at 135.2 100) (size 0.6) (drill 0.3) (layers "F.Cu" "B.Cu") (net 8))
 (segment (start 134.6 100) (end 133.3 98.7) (width 0.2) (layer "B.Cu") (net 8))
 (segment (start 135.2 100) (end 134.6 100) (width 0.2) (layer "B.Cu") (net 8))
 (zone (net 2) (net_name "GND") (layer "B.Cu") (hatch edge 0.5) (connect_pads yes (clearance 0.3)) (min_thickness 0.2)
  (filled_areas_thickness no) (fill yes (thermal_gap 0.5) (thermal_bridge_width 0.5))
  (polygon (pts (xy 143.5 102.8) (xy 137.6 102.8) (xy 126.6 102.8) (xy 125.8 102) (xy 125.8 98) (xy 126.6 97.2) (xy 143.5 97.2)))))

